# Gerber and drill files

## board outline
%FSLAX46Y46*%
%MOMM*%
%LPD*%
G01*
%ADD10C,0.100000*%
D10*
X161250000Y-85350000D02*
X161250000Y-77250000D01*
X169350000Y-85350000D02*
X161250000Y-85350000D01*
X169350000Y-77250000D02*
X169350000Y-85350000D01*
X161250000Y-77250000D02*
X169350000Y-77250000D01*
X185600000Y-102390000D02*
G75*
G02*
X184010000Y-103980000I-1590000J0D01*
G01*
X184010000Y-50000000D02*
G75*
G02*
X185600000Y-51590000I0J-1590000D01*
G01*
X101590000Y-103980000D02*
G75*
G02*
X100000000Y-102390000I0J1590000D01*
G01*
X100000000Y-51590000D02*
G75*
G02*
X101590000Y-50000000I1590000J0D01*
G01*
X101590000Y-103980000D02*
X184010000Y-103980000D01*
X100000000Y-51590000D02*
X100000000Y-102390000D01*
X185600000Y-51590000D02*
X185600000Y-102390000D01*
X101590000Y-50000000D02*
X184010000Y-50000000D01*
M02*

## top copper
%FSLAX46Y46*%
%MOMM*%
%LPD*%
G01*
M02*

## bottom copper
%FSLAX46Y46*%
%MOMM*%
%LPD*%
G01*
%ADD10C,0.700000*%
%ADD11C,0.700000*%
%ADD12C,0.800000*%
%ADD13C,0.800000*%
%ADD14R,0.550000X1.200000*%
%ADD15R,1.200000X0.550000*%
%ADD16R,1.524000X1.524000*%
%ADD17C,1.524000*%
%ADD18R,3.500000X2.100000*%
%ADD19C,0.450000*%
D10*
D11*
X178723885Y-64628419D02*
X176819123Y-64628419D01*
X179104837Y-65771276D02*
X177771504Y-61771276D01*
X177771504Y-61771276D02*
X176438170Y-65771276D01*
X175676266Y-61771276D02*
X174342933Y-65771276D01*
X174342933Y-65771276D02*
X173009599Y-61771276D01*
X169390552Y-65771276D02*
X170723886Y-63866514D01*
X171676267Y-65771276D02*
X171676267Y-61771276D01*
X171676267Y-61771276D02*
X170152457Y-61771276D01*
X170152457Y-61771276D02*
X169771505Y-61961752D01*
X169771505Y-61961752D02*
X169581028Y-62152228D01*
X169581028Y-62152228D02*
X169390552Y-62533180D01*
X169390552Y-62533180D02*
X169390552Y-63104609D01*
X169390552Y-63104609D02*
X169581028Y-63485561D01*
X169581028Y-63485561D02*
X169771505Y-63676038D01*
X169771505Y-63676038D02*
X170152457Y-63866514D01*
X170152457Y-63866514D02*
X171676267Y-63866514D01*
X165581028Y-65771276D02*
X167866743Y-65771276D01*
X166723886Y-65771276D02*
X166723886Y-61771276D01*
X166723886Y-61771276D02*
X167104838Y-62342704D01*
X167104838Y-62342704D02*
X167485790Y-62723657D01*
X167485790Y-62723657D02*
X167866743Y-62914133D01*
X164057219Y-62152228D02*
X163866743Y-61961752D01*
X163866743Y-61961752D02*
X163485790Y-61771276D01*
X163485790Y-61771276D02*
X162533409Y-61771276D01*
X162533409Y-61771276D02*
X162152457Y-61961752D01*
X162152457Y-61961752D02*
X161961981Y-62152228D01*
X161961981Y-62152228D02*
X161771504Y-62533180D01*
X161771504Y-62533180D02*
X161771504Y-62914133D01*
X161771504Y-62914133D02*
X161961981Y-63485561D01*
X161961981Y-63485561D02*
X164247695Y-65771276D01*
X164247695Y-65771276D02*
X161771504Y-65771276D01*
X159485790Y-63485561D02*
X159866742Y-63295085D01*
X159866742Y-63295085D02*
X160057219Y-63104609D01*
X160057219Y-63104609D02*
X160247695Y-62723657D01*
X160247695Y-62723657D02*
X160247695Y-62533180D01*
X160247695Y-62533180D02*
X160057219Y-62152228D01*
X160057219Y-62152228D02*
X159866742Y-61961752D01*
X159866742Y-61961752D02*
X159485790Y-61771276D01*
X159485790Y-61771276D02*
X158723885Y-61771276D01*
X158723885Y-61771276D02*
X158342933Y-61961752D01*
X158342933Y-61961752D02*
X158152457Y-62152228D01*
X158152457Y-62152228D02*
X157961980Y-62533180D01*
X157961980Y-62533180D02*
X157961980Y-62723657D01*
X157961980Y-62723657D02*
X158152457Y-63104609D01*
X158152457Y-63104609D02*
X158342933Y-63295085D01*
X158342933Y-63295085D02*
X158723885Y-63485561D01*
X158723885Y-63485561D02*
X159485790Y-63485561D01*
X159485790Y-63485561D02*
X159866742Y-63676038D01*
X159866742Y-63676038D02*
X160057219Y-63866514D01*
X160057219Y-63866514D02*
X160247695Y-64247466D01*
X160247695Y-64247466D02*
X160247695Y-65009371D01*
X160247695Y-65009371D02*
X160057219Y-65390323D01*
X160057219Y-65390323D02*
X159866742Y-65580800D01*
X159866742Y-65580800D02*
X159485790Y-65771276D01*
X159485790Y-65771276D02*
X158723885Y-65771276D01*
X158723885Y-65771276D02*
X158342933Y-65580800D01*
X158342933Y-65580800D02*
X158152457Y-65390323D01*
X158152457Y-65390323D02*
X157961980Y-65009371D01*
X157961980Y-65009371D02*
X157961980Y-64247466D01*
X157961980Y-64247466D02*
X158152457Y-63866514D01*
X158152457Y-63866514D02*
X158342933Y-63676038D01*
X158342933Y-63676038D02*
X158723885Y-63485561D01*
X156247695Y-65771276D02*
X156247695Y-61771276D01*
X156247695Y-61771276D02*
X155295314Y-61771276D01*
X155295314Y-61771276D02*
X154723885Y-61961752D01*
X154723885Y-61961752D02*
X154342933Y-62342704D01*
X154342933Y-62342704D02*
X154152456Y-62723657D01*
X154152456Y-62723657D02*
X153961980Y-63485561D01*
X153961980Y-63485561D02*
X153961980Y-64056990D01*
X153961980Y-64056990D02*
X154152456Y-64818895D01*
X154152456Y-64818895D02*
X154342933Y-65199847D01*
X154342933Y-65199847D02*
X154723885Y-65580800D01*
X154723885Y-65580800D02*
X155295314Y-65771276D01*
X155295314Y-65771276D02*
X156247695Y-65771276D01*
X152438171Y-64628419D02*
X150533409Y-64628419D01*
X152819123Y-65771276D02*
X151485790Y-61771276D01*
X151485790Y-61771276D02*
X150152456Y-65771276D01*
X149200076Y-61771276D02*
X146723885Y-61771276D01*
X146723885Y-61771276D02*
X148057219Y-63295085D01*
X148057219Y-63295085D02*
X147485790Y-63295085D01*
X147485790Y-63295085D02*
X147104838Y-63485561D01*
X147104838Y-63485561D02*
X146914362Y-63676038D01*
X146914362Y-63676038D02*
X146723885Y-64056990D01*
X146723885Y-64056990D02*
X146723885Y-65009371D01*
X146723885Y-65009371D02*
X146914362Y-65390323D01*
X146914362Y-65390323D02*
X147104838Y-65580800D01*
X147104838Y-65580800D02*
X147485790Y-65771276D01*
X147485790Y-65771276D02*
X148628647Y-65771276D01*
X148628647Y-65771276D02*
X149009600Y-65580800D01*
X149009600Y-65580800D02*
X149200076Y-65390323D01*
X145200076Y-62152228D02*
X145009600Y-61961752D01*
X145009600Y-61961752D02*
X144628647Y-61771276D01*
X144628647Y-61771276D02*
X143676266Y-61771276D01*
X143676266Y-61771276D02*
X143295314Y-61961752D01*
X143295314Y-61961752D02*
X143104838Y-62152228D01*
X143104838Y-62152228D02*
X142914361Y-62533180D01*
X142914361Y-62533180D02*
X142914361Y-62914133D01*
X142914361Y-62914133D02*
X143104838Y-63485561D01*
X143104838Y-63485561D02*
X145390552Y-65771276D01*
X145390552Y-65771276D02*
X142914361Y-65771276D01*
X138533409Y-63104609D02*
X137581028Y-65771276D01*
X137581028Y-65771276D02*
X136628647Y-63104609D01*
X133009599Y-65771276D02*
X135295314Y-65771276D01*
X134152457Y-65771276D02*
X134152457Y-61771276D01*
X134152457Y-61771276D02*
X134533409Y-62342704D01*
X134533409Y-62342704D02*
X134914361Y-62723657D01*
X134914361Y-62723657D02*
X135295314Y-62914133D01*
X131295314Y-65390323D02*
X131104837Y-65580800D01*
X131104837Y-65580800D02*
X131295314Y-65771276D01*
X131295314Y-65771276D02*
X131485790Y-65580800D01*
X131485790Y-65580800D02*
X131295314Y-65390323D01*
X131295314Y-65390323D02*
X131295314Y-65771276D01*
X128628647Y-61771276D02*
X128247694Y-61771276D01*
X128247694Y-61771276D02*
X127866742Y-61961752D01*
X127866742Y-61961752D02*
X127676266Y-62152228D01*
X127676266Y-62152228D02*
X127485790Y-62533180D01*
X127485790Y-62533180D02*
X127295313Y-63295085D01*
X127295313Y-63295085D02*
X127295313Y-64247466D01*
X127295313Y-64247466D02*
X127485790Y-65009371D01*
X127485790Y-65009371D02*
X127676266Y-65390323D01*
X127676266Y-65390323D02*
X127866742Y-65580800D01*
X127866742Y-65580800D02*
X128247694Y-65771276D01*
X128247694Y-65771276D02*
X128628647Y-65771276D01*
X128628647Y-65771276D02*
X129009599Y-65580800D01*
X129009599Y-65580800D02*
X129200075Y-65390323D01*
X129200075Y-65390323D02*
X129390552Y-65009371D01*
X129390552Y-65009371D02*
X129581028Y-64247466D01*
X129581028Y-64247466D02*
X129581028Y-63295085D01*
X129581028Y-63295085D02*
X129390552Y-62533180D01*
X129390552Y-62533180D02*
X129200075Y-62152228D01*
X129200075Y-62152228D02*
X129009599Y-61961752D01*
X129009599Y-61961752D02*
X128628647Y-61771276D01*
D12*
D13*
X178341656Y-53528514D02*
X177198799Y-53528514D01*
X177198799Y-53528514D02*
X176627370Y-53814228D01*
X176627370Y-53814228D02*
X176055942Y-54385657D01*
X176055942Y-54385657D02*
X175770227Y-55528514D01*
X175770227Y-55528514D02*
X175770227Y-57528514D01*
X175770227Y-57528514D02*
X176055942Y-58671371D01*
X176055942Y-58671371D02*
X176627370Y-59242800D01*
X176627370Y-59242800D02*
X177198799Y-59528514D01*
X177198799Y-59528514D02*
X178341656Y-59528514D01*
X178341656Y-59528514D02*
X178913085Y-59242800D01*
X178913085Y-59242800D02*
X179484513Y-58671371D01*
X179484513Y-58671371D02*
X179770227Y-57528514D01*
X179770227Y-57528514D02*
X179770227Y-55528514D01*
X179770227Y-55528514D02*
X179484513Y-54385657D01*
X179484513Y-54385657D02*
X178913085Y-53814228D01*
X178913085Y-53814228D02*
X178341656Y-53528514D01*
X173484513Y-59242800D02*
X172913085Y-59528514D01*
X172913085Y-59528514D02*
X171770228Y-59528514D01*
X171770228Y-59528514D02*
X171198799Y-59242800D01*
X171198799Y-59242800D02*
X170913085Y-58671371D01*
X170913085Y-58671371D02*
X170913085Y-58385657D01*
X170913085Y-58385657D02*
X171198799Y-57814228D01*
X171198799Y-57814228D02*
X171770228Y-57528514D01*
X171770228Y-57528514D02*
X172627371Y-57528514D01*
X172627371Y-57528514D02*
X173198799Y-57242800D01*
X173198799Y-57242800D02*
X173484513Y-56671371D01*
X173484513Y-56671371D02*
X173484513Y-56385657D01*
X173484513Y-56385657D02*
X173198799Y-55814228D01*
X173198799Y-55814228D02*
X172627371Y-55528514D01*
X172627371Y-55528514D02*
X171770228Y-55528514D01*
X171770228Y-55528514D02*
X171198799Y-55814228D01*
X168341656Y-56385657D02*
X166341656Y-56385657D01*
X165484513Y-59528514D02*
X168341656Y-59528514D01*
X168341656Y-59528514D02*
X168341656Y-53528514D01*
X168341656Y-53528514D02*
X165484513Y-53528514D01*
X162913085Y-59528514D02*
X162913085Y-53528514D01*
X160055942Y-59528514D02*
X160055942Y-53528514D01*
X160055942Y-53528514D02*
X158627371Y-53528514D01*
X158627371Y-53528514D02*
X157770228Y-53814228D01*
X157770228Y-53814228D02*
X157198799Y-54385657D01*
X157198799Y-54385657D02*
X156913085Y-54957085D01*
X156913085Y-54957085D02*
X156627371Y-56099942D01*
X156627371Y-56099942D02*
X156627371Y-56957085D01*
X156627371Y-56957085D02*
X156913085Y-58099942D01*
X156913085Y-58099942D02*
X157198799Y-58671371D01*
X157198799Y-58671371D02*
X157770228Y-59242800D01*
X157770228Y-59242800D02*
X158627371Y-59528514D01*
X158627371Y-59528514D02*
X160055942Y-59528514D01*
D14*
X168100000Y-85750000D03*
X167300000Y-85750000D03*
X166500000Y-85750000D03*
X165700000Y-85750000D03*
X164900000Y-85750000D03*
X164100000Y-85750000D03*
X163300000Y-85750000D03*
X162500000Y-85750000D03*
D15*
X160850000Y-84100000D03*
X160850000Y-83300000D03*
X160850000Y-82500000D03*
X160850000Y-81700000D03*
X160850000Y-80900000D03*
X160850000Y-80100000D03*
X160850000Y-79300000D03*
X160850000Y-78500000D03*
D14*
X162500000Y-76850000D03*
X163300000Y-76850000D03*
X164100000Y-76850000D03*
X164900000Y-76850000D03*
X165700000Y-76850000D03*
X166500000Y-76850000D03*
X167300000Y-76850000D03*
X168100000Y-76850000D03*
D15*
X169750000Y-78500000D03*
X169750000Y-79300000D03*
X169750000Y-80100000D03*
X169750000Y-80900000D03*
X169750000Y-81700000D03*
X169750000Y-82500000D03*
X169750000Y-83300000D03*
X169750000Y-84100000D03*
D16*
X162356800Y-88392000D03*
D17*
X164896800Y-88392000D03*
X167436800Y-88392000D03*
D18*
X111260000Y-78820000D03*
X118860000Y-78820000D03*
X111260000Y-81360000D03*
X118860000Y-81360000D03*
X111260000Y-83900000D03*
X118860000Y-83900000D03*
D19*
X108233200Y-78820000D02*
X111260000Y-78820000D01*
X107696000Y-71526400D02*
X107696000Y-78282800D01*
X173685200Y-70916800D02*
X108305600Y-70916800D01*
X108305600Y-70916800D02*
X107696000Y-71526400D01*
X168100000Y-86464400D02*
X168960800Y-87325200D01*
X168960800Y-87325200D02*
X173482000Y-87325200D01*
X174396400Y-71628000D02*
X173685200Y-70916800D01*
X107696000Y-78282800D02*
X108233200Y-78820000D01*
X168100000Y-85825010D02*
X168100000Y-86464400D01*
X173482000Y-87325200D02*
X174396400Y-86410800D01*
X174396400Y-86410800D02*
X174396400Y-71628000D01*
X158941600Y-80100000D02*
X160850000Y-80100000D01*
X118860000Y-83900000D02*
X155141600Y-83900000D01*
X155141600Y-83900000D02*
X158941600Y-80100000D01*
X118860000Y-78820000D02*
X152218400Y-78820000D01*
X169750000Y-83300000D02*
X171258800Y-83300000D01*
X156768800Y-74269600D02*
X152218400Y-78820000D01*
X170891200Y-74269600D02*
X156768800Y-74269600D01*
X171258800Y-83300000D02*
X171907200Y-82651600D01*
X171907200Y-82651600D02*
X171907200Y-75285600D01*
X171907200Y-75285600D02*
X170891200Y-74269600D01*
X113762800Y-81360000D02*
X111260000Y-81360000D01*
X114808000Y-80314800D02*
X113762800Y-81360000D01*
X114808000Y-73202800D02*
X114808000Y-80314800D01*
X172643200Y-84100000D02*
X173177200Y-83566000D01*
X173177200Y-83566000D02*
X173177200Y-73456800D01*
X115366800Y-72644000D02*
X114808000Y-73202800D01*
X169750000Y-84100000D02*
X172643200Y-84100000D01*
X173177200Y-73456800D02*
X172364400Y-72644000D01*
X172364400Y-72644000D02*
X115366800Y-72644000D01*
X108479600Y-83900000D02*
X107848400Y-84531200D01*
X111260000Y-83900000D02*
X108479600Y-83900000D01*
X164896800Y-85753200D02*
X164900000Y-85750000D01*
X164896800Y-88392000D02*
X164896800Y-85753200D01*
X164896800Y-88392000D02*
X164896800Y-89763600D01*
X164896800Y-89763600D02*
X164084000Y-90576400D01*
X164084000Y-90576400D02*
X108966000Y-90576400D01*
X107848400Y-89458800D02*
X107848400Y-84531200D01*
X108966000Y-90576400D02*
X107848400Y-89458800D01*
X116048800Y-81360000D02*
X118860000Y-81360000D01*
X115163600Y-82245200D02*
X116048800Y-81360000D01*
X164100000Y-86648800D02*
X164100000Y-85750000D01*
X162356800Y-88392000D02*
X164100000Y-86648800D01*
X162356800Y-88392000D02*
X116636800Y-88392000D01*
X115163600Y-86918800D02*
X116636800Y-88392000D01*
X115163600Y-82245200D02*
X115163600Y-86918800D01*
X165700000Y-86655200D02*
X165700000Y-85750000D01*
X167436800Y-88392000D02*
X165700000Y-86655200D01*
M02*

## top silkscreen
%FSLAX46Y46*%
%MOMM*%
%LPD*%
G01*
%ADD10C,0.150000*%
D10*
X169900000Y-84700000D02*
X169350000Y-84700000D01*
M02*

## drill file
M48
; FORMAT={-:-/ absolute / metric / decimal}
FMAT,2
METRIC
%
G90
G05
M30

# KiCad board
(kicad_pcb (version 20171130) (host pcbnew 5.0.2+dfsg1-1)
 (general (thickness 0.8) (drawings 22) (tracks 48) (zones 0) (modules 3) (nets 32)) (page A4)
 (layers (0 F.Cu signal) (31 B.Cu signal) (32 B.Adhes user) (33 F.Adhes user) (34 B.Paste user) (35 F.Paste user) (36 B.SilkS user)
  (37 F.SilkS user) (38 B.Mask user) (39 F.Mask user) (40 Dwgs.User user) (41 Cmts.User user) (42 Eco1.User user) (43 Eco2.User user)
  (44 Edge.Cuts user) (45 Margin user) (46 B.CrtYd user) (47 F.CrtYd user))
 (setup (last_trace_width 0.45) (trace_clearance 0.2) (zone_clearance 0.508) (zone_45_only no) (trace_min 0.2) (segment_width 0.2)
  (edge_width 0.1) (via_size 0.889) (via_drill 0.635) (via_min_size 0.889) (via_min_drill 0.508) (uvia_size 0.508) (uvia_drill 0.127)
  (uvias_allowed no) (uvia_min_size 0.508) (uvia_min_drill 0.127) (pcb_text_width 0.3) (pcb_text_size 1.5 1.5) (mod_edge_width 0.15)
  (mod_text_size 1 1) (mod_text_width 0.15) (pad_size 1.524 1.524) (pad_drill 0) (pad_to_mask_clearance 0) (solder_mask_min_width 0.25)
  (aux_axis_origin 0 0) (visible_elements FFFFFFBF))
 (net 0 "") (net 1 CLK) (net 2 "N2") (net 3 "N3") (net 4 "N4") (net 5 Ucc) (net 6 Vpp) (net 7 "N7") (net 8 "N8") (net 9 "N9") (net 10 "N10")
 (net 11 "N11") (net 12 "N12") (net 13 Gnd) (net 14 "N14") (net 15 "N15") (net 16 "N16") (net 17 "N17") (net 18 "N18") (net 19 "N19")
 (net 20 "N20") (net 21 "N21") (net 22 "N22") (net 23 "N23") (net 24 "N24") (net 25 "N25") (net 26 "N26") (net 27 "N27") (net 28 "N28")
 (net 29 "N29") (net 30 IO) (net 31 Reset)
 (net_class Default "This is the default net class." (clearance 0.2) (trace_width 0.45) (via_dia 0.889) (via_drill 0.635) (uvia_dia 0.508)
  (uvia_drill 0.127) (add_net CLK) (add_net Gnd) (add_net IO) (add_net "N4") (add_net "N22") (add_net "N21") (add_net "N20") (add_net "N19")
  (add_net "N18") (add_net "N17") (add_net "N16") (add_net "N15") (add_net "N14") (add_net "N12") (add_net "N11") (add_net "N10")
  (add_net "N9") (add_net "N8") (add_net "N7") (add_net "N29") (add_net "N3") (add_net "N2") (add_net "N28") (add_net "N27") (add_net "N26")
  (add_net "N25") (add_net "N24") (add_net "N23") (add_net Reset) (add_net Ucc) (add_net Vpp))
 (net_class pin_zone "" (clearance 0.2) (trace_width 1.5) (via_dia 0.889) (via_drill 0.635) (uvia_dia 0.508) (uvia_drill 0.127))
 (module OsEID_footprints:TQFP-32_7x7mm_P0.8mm (layer F.Cu) (at 165.3 81.3 180)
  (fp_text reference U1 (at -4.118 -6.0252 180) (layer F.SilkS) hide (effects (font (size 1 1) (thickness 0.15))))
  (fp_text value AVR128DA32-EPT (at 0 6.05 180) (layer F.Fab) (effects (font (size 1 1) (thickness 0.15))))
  (fp_line (start -4.6 -3.4) (end -4.05 -3.4) (layer F.SilkS) (width 0.15))
  (pad 32 smd rect (at -2.8 -4.45 270) (size 1.2 0.55) (layers B.Cu B.Paste B.Mask) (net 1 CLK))
  (pad 31 smd rect (at -2 -4.45 270) (size 1.2 0.55) (layers B.Cu B.Paste B.Mask) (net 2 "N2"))
  (pad 30 smd rect (at -1.2 -4.45 270) (size 1.2 0.55) (layers B.Cu B.Paste B.Mask) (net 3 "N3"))
  (pad 29 smd rect (at -0.4 -4.45 270) (size 1.2 0.55) (layers B.Cu B.Paste B.Mask) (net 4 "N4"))
  (pad 28 smd rect (at 0.4 -4.45 270) (size 1.2 0.55) (layers B.Cu B.Paste B.Mask) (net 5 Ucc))
  (pad 27 smd rect (at 1.2 -4.45 270) (size 1.2 0.55) (layers B.Cu B.Paste B.Mask) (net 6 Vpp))
  (pad 26 smd rect (at 2 -4.45 270) (size 1.2 0.55) (layers B.Cu B.Paste B.Mask) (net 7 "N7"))
  (pad 25 smd rect (at 2.8 -4.45 270) (size 1.2 0.55) (layers B.Cu B.Paste B.Mask) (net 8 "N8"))
  (pad 24 smd rect (at 4.45 -2.8 180) (size 1.2 0.55) (layers B.Cu B.Paste B.Mask) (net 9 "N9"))
  (pad 23 smd rect (at 4.45 -2 180) (size 1.2 0.55) (layers B.Cu B.Paste B.Mask))
  (pad 22 smd rect (at 4.45 -1.2 180) (size 1.2 0.55) (layers B.Cu B.Paste B.Mask) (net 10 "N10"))
  (pad 21 smd rect (at 4.45 -0.4 180) (size 1.2 0.55) (layers B.Cu B.Paste B.Mask) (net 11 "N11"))
  (pad 20 smd rect (at 4.45 0.4 180) (size 1.2 0.55) (layers B.Cu B.Paste B.Mask) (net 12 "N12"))
  (pad 19 smd rect (at 4.45 1.2 180) (size 1.2 0.55) (layers B.Cu B.Paste B.Mask) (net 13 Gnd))
  (pad 18 smd rect (at 4.45 2 180) (size 1.2 0.55) (layers B.Cu B.Paste B.Mask) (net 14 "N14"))
  (pad 17 smd rect (at 4.45 2.8 180) (size 1.2 0.55) (layers B.Cu B.Paste B.Mask) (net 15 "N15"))
  (pad 16 smd rect (at 2.8 4.45 270) (size 1.2 0.55) (layers B.Cu B.Paste B.Mask) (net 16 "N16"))
  (pad 15 smd rect (at 2 4.45 270) (size 1.2 0.55) (layers B.Cu B.Paste B.Mask) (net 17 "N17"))
  (pad 14 smd rect (at 1.2 4.45 270) (size 1.2 0.55) (layers B.Cu B.Paste B.Mask) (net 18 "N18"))
  (pad 13 smd rect (at 0.4 4.45 270) (size 1.2 0.55) (layers B.Cu B.Paste B.Mask) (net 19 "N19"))
  (pad 12 smd rect (at -0.4 4.45 270) (size 1.2 0.55) (layers B.Cu B.Paste B.Mask) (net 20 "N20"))
  (pad 11 smd rect (at -1.2 4.45 270) (size 1.2 0.55) (layers B.Cu B.Paste B.Mask) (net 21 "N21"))
  (pad 10 smd rect (at -2 4.45 270) (size 1.2 0.55) (layers B.Cu B.Paste B.Mask) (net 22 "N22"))
  (pad 9 smd rect (at -2.8 4.45 270) (size 1.2 0.55) (layers B.Cu B.Paste B.Mask) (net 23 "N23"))
  (pad 8 smd rect (at -4.45 2.8 180) (size 1.2 0.55) (layers B.Cu B.Paste B.Mask) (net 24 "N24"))
  (pad 7 smd rect (at -4.45 2 180) (size 1.2 0.55) (layers B.Cu B.Paste B.Mask) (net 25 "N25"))
  (pad 6 smd rect (at -4.45 1.2 180) (size 1.2 0.55) (layers B.Cu B.Paste B.Mask) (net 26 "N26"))
  (pad 5 smd rect (at -4.45 0.4 180) (size 1.2 0.55) (layers B.Cu B.Paste B.Mask) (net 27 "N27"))
  (pad 4 smd rect (at -4.45 -0.4 180) (size 1.2 0.55) (layers B.Cu B.Paste B.Mask) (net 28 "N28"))
  (pad 3 smd rect (at -4.45 -1.2 180) (size 1.2 0.55) (layers B.Cu B.Paste B.Mask) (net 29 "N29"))
  (pad 2 smd rect (at -4.45 -2 180) (size 1.2 0.55) (layers B.Cu B.Paste B.Mask) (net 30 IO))
  (pad 1 smd rect (at -4.45 -2.8 180) (size 1.2 0.55) (layers B.Cu B.Paste B.Mask) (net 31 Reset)))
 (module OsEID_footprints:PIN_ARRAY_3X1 (layer F.Cu) (at 164.8968 88.392)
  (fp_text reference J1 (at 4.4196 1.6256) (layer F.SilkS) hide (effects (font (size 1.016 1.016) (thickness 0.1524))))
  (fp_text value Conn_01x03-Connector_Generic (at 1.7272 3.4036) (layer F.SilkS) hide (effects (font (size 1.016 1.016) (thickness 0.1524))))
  (pad 1 connect rect (at -2.54 0) (size 1.524 1.524) (layers B.Cu B.Mask) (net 6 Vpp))
  (pad 2 connect circle (at 0 0) (size 1.524 1.524) (layers B.Cu B.Mask) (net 5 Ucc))
  (pad 3 connect circle (at 2.54 0) (size 1.524 1.524) (layers B.Cu B.Mask) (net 4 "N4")))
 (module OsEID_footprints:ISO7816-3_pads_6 (layer B.Cu) (at 115.06 81.36 90)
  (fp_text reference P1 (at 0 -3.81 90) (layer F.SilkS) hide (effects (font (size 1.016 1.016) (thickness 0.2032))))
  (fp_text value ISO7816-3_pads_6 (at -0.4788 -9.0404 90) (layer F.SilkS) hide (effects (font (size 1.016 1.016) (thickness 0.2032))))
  (pad 6 smd rect (at 2.54 -3.8 90) (size 2.1 3.5) (layers B.Cu B.Mask) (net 1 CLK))
  (pad 5 smd rect (at 2.54 3.8 90) (size 2.1 3.5) (layers B.Cu B.Mask) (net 30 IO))
  (pad 4 smd rect (at 0 -3.8 90) (size 2.1 3.5) (layers B.Cu B.Mask) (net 31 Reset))
  (pad 3 smd rect (at 0 3.8 90) (size 2.1 3.5) (layers B.Cu B.Mask) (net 6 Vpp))
  (pad 2 smd rect (at -2.54 -3.8 90) (size 2.1 3.5) (layers B.Cu B.Mask) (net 5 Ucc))
  (pad 1 smd rect (at -2.54 3.8 90) (size 2.1 3.5) (layers B.Cu B.Mask) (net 13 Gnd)))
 (gr_line (start 161.25 85.35) (end 161.25 77.25) (layer Edge.Cuts) (width 0.1))
 (gr_line (start 169.35 85.35) (end 161.25 85.35) (layer Edge.Cuts) (width 0.1))
 (gr_line (start 169.35 77.25) (end 169.35 85.35) (layer Edge.Cuts) (width 0.1))
 (gr_line (start 161.25 77.25) (end 169.35 77.25) (layer Edge.Cuts) (width 0.1))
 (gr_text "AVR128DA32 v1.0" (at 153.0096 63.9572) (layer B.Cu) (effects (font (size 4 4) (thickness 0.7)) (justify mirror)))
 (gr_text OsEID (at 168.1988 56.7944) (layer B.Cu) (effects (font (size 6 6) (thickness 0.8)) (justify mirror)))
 (gr_arc (start 184.01 102.39) (end 185.6 102.39) (angle 90) (layer Edge.Cuts) (width 0.1))
 (gr_arc (start 184.01 51.59) (end 184.01 50) (angle 90) (layer Edge.Cuts) (width 0.1))
 (gr_arc (start 101.59 102.39) (end 101.59 103.98) (angle 90) (layer Edge.Cuts) (width 0.1))
 (gr_arc (start 101.59 51.59) (end 100 51.59) (angle 90) (layer Edge.Cuts) (width 0.1))
 (gr_line (start 101.59 103.98) (end 184.01 103.98) (angle 90) (layer Edge.Cuts) (width 0.1))
 (gr_line (start 100 51.59) (end 100 102.39) (angle 90) (layer Edge.Cuts) (width 0.1))
 (gr_line (start 185.6 51.59) (end 185.6 102.39) (angle 90) (layer Edge.Cuts) (width 0.1))
 (gr_line (start 101.59 50) (end 184.01 50) (angle 90) (layer Edge.Cuts) (width 0.1))
 (segment (start 108.2332 78.82) (end 111.26 78.82) (width 0.45) (layer B.Cu) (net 1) (status 20))
 (segment (start 107.696 71.5264) (end 107.696 78.2828) (width 0.45) (layer B.Cu) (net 1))
 (segment (start 173.6852 70.9168) (end 108.3056 70.9168) (width 0.45) (layer B.Cu) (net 1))
 (segment (start 108.3056 70.9168) (end 107.696 71.5264) (width 0.45) (layer B.Cu) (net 1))
 (segment (start 168.1 86.4644) (end 168.9608 87.3252) (width 0.45) (layer B.Cu) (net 1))
 (segment (start 168.9608 87.3252) (end 173.482 87.3252) (width 0.45) (layer B.Cu) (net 1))
 (segment (start 174.3964 71.628) (end 173.6852 70.9168) (width 0.45) (layer B.Cu) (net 1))
 (segment (start 107.696 78.2828) (end 108.2332 78.82) (width 0.45) (layer B.Cu) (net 1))
 (segment (start 168.1 85.82501) (end 168.1 86.4644) (width 0.45) (layer B.Cu) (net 1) (status 10))
 (segment (start 173.482 87.3252) (end 174.3964 86.4108) (width 0.45) (layer B.Cu) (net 1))
 (segment (start 174.3964 86.4108) (end 174.3964 71.628) (width 0.45) (layer B.Cu) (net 1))
 (segment (start 158.9416 80.1) (end 160.85 80.1) (width 0.45) (layer B.Cu) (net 13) (status 20))
 (segment (start 118.86 83.9) (end 155.1416 83.9) (width 0.45) (layer B.Cu) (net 13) (status 10))
 (segment (start 155.1416 83.9) (end 158.9416 80.1) (width 0.45) (layer B.Cu) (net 13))
 (segment (start 118.86 78.82) (end 152.2184 78.82) (width 0.45) (layer B.Cu) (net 30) (status 10))
 (segment (start 169.75 83.3) (end 171.2588 83.3) (width 0.45) (layer B.Cu) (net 30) (status 10))
 (segment (start 156.7688 74.2696) (end 152.2184 78.82) (width 0.45) (layer B.Cu) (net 30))
 (segment (start 170.8912 74.2696) (end 156.7688 74.2696) (width 0.45) (layer B.Cu) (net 30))
 (segment (start 171.2588 83.3) (end 171.9072 82.6516) (width 0.45) (layer B.Cu) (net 30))
 (segment (start 171.9072 82.6516) (end 171.9072 75.2856) (width 0.45) (layer B.Cu) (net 30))
 (segment (start 171.9072 75.2856) (end 170.8912 74.2696) (width 0.45) (layer B.Cu) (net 30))
 (segment (start 113.7628 81.36) (end 111.26 81.36) (width 0.45) (layer B.Cu) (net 31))
 (segment (start 114.808 80.3148) (end 113.7628 81.36) (width 0.45) (layer B.Cu) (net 31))
 (segment (start 114.808 73.2028) (end 114.808 80.3148) (width 0.45) (layer B.Cu) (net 31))
 (segment (start 172.6432 84.1) (end 173.1772 83.566) (width 0.45) (layer B.Cu) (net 31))
 (segment (start 173.1772 83.566) (end 173.1772 73.4568) (width 0.45) (layer B.Cu) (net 31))
 (segment (start 115.3668 72.644) (end 114.808 73.2028) (width 0.45) (layer B.Cu) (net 31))
 (segment (start 169.75 84.1) (end 172.6432 84.1) (width 0.45) (layer B.Cu) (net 31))
 (segment (start 173.1772 73.4568) (end 172.3644 72.644) (width 0.45) (layer B.Cu) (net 31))
 (segment (start 172.3644 72.644) (end 115.3668 72.644) (width 0.45) (layer B.Cu) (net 31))
 (segment (start 108.4796 83.9) (end 107.8484 84.5312) (width 0.45) (layer B.Cu) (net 5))
 (segment (start 111.26 83.9) (end 108.4796 83.9) (width 0.45) (layer B.Cu) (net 5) (status 10))
 (segment (start 164.8968 85.7532) (end 164.9 85.75) (width 0.45) (layer B.Cu) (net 5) (status 30))
 (segment (start 164.8968 88.392) (end 164.8968 85.7532) (width 0.45) (layer B.Cu) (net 5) (status 30))
 (segment (start 164.8968 88.392) (end 164.8968 89.7636) (width 0.45) (layer B.Cu) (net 5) (status 10))
 (segment (start 164.8968 89.7636) (end 164.084 90.5764) (width 0.45) (layer B.Cu) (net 5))
 (segment (start 164.084 90.5764) (end 108.966 90.5764) (width 0.45) (layer B.Cu) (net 5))
 (segment (start 107.8484 89.4588) (end 107.8484 84.5312) (width 0.45) (layer B.Cu) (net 5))
 (segment (start 108.966 90.5764) (end 107.8484 89.4588) (width 0.45) (layer B.Cu) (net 5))
 (segment (start 116.0488 81.36) (end 118.86 81.36) (width 0.45) (layer B.Cu) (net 6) (status 20))
 (segment (start 115.1636 82.2452) (end 116.0488 81.36) (width 0.45) (layer B.Cu) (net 6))
 (segment (start 164.1 86.6488) (end 164.1 85.75) (width 0.45) (layer B.Cu) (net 6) (status 20))
 (segment (start 162.3568 88.392) (end 164.1 86.6488) (width 0.45) (layer B.Cu) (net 6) (status 10))
 (segment (start 162.3568 88.392) (end 116.6368 88.392) (width 0.45) (layer B.Cu) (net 6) (status 10))
 (segment (start 115.1636 86.9188) (end 116.6368 88.392) (width 0.45) (layer B.Cu) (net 6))
 (segment (start 115.1636 82.2452) (end 115.1636 86.9188) (width 0.45) (layer B.Cu) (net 6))
 (segment (start 165.7 86.6552) (end 165.7 85.75) (width 0.45) (layer B.Cu) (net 4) (status 20))
 (segment (start 167.4368 88.392) (end 165.7 86.6552) (width 0.45) (layer B.Cu) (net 4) (status 10)))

